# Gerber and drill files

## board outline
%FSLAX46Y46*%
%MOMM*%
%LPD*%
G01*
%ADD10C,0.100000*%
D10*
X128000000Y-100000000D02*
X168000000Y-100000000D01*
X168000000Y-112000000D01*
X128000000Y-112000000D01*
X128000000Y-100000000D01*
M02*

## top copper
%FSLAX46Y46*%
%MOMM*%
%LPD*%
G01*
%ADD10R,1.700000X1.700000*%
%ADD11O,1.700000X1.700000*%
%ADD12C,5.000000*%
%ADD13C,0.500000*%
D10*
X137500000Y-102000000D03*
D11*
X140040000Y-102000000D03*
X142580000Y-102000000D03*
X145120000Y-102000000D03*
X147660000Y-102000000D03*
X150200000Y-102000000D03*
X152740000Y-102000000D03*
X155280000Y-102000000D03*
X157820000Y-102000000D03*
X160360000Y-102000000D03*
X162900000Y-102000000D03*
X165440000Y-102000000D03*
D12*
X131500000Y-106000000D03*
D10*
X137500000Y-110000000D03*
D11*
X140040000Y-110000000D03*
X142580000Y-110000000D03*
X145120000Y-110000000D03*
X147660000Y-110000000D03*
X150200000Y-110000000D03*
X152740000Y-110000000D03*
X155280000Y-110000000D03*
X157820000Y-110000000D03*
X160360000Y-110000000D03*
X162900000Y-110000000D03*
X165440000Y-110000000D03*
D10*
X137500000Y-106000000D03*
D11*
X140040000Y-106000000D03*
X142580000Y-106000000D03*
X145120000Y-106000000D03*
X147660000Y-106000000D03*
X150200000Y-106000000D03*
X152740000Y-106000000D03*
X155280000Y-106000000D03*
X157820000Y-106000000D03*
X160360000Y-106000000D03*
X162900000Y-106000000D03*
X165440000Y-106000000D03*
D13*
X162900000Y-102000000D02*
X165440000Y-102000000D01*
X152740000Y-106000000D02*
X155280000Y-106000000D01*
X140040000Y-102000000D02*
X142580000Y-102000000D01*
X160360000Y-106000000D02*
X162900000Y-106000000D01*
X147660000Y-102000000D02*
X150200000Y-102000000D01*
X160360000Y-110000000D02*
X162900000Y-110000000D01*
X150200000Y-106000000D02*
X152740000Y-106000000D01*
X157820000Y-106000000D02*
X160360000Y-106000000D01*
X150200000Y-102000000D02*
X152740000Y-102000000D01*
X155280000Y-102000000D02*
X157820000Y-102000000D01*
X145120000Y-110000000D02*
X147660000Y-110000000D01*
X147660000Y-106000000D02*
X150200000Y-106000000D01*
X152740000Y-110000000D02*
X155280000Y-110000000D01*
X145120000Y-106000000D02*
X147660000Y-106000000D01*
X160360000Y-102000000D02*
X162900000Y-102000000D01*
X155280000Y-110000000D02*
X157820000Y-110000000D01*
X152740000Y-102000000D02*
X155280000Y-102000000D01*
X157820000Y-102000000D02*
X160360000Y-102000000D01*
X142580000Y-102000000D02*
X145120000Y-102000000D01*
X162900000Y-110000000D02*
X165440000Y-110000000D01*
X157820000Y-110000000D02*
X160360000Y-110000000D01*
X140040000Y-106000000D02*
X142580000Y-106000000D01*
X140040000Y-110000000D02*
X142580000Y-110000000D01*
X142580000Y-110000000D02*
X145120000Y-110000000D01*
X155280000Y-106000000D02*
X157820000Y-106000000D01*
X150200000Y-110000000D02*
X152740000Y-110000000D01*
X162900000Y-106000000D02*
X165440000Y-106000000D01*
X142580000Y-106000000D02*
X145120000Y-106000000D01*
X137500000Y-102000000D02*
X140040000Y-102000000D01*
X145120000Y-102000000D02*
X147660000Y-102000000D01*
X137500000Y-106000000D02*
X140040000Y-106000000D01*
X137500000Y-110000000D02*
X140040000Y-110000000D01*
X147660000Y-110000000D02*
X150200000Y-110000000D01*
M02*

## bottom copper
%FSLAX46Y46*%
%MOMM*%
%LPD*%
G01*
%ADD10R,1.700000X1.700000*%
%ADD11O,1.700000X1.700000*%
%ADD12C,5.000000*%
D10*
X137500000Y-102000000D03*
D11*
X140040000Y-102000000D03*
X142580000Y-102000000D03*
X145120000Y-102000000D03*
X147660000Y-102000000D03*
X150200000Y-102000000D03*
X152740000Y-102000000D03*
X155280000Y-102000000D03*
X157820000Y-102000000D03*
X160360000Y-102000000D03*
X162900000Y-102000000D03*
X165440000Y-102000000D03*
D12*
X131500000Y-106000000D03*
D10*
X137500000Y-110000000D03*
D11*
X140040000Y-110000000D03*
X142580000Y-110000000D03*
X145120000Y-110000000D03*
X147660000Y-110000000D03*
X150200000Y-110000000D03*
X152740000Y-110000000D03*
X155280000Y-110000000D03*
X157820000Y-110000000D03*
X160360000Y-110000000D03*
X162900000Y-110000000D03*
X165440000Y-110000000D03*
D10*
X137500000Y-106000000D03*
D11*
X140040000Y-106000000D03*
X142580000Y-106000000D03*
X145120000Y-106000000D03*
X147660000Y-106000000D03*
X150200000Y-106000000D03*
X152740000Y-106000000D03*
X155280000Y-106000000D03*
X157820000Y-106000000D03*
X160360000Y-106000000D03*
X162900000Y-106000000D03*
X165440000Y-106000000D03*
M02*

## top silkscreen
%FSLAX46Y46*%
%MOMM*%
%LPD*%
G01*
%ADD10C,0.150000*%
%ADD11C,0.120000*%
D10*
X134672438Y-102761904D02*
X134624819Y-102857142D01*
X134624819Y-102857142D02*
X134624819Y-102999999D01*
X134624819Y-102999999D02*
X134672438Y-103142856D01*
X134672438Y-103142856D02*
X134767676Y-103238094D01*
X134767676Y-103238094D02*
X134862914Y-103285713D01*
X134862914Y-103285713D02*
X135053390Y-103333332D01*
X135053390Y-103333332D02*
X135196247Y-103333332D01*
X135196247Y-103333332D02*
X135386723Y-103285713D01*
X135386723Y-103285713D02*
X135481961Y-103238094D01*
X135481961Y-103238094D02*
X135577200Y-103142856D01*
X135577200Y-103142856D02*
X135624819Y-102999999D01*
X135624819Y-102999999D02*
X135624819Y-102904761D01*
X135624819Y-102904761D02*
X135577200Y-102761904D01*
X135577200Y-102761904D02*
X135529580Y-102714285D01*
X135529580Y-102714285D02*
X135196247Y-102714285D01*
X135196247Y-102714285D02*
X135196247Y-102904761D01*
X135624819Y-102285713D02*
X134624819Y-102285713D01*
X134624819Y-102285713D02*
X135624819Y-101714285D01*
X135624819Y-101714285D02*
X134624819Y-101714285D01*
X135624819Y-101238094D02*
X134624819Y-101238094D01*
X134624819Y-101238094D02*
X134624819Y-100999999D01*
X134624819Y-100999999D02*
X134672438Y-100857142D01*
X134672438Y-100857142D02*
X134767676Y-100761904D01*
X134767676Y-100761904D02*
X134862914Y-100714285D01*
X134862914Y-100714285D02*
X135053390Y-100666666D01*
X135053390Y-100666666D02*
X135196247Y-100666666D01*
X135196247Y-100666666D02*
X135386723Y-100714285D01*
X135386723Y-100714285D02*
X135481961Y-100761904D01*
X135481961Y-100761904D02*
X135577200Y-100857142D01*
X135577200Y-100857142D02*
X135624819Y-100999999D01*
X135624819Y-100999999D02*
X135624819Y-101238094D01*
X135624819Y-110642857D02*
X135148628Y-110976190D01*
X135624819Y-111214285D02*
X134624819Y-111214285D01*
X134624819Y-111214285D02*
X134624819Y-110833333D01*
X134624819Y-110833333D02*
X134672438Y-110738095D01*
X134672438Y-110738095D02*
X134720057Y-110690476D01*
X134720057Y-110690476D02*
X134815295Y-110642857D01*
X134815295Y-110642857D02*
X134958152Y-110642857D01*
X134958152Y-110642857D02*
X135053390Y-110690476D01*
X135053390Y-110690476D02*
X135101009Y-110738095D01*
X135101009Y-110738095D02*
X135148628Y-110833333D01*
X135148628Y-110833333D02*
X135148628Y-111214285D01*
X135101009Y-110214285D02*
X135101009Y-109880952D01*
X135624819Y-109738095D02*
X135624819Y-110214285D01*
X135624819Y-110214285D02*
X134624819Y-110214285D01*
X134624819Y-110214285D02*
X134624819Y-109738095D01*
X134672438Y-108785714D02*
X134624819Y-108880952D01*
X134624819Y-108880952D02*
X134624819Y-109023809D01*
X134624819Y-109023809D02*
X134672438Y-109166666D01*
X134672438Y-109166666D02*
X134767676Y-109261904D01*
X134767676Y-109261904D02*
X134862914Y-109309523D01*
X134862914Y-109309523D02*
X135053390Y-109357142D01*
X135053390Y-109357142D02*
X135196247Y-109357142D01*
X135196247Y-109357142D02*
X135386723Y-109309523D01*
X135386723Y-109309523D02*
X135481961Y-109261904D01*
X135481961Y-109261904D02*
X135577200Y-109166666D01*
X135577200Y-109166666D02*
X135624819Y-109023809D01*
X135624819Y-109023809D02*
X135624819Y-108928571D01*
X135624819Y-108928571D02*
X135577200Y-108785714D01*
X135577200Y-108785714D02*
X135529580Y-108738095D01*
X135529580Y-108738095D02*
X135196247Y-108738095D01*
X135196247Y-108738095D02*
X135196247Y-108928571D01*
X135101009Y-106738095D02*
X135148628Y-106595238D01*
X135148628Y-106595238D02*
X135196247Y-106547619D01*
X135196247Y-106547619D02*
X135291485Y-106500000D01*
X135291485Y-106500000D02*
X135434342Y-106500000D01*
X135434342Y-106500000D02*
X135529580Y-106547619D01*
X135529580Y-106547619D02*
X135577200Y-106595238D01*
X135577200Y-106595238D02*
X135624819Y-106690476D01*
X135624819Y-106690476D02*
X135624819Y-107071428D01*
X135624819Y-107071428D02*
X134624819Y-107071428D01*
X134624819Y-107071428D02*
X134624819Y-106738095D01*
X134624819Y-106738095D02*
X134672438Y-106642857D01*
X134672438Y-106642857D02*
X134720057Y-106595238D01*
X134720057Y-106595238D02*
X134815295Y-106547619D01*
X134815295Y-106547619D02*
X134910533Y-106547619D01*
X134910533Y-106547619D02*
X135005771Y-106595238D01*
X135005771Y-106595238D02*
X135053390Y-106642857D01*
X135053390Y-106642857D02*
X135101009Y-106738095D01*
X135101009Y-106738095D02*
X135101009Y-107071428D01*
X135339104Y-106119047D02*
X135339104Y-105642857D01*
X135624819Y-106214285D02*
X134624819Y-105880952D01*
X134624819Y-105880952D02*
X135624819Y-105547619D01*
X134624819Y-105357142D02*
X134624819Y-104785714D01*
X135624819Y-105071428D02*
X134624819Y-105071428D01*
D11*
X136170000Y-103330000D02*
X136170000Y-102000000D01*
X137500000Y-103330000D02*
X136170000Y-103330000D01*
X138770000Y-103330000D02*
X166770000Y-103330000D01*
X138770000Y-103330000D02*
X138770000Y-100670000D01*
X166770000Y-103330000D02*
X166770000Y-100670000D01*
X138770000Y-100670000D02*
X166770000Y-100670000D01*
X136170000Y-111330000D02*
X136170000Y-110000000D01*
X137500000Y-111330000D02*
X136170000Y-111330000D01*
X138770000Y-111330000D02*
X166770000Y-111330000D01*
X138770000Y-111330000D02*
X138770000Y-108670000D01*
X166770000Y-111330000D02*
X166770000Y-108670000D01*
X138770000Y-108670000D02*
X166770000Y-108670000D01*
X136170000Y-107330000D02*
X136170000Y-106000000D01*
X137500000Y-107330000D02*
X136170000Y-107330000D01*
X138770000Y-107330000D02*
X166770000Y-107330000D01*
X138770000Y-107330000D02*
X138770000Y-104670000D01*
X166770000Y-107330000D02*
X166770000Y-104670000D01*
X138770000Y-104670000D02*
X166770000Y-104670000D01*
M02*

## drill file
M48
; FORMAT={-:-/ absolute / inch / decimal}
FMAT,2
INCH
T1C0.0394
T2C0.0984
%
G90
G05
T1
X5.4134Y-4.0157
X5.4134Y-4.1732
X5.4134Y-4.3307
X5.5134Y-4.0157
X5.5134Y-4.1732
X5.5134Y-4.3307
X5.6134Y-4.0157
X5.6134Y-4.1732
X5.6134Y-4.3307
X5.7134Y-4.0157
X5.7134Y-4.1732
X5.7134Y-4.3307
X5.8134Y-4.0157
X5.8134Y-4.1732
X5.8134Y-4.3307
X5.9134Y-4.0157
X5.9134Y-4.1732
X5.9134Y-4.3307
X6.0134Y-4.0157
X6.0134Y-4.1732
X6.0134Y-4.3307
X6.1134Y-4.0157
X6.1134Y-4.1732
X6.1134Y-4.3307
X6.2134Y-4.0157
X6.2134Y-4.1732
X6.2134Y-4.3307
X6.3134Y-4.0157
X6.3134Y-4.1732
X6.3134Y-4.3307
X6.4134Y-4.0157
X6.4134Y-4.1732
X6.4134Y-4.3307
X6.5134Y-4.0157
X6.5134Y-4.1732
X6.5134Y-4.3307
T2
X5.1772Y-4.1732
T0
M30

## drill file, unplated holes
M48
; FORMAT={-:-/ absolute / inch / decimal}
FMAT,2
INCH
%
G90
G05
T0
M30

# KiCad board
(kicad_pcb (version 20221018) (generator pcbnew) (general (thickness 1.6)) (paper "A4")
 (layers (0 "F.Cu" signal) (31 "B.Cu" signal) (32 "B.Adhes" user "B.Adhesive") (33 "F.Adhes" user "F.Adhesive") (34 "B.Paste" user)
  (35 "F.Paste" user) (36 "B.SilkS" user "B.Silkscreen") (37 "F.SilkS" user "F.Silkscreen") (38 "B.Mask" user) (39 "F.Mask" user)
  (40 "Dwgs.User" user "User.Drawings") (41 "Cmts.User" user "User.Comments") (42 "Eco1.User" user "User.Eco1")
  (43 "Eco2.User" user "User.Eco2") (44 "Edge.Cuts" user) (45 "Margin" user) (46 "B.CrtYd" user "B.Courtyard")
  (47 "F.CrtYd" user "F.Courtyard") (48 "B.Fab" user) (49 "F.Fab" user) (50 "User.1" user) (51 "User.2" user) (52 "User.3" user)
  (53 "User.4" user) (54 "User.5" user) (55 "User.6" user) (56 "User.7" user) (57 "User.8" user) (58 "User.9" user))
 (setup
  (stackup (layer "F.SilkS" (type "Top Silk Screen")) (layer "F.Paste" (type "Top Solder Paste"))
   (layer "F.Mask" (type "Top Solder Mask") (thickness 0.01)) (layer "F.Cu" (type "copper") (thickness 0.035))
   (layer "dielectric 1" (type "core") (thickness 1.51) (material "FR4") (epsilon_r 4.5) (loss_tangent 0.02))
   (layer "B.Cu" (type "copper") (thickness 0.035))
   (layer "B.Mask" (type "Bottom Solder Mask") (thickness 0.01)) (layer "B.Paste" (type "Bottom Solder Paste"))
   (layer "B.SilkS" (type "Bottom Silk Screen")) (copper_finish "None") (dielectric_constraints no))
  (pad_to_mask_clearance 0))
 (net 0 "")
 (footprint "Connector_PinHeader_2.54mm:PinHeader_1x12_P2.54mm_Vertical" (layer "F.Cu") (at 137.5 102 90)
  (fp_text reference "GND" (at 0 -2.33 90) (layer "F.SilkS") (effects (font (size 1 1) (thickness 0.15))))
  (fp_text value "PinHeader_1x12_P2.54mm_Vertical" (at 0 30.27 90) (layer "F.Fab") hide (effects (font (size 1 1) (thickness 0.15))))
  (fp_line (start -1.33 -1.33) (end 0 -1.33) (stroke (width 0.12) (type solid)) (layer "F.SilkS"))
  (fp_line (start -1.33 0) (end -1.33 -1.33) (stroke (width 0.12) (type solid)) (layer "F.SilkS"))
  (fp_line (start -1.33 1.27) (end -1.33 29.27) (stroke (width 0.12) (type solid)) (layer "F.SilkS"))
  (fp_line (start -1.33 1.27) (end 1.33 1.27) (stroke (width 0.12) (type solid)) (layer "F.SilkS"))
  (fp_line (start -1.33 29.27) (end 1.33 29.27) (stroke (width 0.12) (type solid)) (layer "F.SilkS"))
  (fp_line (start 1.33 1.27) (end 1.33 29.27) (stroke (width 0.12) (type solid)) (layer "F.SilkS"))
  (pad "1" thru_hole rect (at 0 0 90) (size 1.7 1.7) (drill 1) (layers "*.Cu" "*.Mask"))
  (pad "2" thru_hole oval (at 0 2.54 90) (size 1.7 1.7) (drill 1) (layers "*.Cu" "*.Mask"))
  (pad "3" thru_hole oval (at 0 5.08 90) (size 1.7 1.7) (drill 1) (layers "*.Cu" "*.Mask"))
  (pad "4" thru_hole oval (at 0 7.62 90) (size 1.7 1.7) (drill 1) (layers "*.Cu" "*.Mask"))
  (pad "5" thru_hole oval (at 0 10.16 90) (size 1.7 1.7) (drill 1) (layers "*.Cu" "*.Mask"))
  (pad "6" thru_hole oval (at 0 12.7 90) (size 1.7 1.7) (drill 1) (layers "*.Cu" "*.Mask"))
  (pad "7" thru_hole oval (at 0 15.24 90) (size 1.7 1.7) (drill 1) (layers "*.Cu" "*.Mask"))
  (pad "8" thru_hole oval (at 0 17.78 90) (size 1.7 1.7) (drill 1) (layers "*.Cu" "*.Mask"))
  (pad "9" thru_hole oval (at 0 20.32 90) (size 1.7 1.7) (drill 1) (layers "*.Cu" "*.Mask"))
  (pad "10" thru_hole oval (at 0 22.86 90) (size 1.7 1.7) (drill 1) (layers "*.Cu" "*.Mask"))
  (pad "11" thru_hole oval (at 0 25.4 90) (size 1.7 1.7) (drill 1) (layers "*.Cu" "*.Mask"))
  (pad "12" thru_hole oval (at 0 27.94 90) (size 1.7 1.7) (drill 1) (layers "*.Cu" "*.Mask")))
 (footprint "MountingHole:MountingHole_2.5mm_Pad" (layer "F.Cu") (at 131.5 106)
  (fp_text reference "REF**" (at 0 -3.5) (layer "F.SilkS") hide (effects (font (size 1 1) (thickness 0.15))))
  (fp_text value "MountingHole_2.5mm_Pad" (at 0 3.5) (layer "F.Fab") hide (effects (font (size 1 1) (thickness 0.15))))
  (pad "1" thru_hole circle (at 0 0) (size 5 5) (drill 2.5) (layers "*.Cu" "*.Mask")))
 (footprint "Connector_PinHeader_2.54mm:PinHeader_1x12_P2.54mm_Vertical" (layer "F.Cu") (at 137.5 110 90)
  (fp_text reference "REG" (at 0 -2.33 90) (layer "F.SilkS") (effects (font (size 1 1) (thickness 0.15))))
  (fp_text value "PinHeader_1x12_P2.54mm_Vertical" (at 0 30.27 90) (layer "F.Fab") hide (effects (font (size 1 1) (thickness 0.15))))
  (fp_line (start -1.33 -1.33) (end 0 -1.33) (stroke (width 0.12) (type solid)) (layer "F.SilkS"))
  (fp_line (start -1.33 0) (end -1.33 -1.33) (stroke (width 0.12) (type solid)) (layer "F.SilkS"))
  (fp_line (start -1.33 1.27) (end -1.33 29.27) (stroke (width 0.12) (type solid)) (layer "F.SilkS"))
  (fp_line (start -1.33 1.27) (end 1.33 1.27) (stroke (width 0.12) (type solid)) (layer "F.SilkS"))
  (fp_line (start -1.33 29.27) (end 1.33 29.27) (stroke (width 0.12) (type solid)) (layer "F.SilkS"))
  (fp_line (start 1.33 1.27) (end 1.33 29.27) (stroke (width 0.12) (type solid)) (layer "F.SilkS"))
  (pad "1" thru_hole rect (at 0 0 90) (size 1.7 1.7) (drill 1) (layers "*.Cu" "*.Mask"))
  (pad "2" thru_hole oval (at 0 2.54 90) (size 1.7 1.7) (drill 1) (layers "*.Cu" "*.Mask"))
  (pad "3" thru_hole oval (at 0 5.08 90) (size 1.7 1.7) (drill 1) (layers "*.Cu" "*.Mask"))
  (pad "4" thru_hole oval (at 0 7.62 90) (size 1.7 1.7) (drill 1) (layers "*.Cu" "*.Mask"))
  (pad "5" thru_hole oval (at 0 10.16 90) (size 1.7 1.7) (drill 1) (layers "*.Cu" "*.Mask"))
  (pad "6" thru_hole oval (at 0 12.7 90) (size 1.7 1.7) (drill 1) (layers "*.Cu" "*.Mask"))
  (pad "7" thru_hole oval (at 0 15.24 90) (size 1.7 1.7) (drill 1) (layers "*.Cu" "*.Mask"))
  (pad "8" thru_hole oval (at 0 17.78 90) (size 1.7 1.7) (drill 1) (layers "*.Cu" "*.Mask"))
  (pad "9" thru_hole oval (at 0 20.32 90) (size 1.7 1.7) (drill 1) (layers "*.Cu" "*.Mask"))
  (pad "10" thru_hole oval (at 0 22.86 90) (size 1.7 1.7) (drill 1) (layers "*.Cu" "*.Mask"))
  (pad "11" thru_hole oval (at 0 25.4 90) (size 1.7 1.7) (drill 1) (layers "*.Cu" "*.Mask"))
  (pad "12" thru_hole oval (at 0 27.94 90) (size 1.7 1.7) (drill 1) (layers "*.Cu" "*.Mask")))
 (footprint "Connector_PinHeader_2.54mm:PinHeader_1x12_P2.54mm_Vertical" (layer "F.Cu") (at 137.5 106 90)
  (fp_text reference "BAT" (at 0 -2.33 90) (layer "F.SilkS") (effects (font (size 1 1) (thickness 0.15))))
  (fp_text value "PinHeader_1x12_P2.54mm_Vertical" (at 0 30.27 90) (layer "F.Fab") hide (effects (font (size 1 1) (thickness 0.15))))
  (fp_line (start -1.33 -1.33) (end 0 -1.33) (stroke (width 0.12) (type solid)) (layer "F.SilkS"))
  (fp_line (start -1.33 0) (end -1.33 -1.33) (stroke (width 0.12) (type solid)) (layer "F.SilkS"))
  (fp_line (start -1.33 1.27) (end -1.33 29.27) (stroke (width 0.12) (type solid)) (layer "F.SilkS"))
  (fp_line (start -1.33 1.27) (end 1.33 1.27) (stroke (width 0.12) (type solid)) (layer "F.SilkS"))
  (fp_line (start -1.33 29.27) (end 1.33 29.27) (stroke (width 0.12) (type solid)) (layer "F.SilkS"))
  (fp_line (start 1.33 1.27) (end 1.33 29.27) (stroke (width 0.12) (type solid)) (layer "F.SilkS"))
  (pad "1" thru_hole rect (at 0 0 90) (size 1.7 1.7) (drill 1) (layers "*.Cu" "*.Mask"))
  (pad "2" thru_hole oval (at 0 2.54 90) (size 1.7 1.7) (drill 1) (layers "*.Cu" "*.Mask"))
  (pad "3" thru_hole oval (at 0 5.08 90) (size 1.7 1.7) (drill 1) (layers "*.Cu" "*.Mask"))
  (pad "4" thru_hole oval (at 0 7.62 90) (size 1.7 1.7) (drill 1) (layers "*.Cu" "*.Mask"))
  (pad "5" thru_hole oval (at 0 10.16 90) (size 1.7 1.7) (drill 1) (layers "*.Cu" "*.Mask"))
  (pad "6" thru_hole oval (at 0 12.7 90) (size 1.7 1.7) (drill 1) (layers "*.Cu" "*.Mask"))
  (pad "7" thru_hole oval (at 0 15.24 90) (size 1.7 1.7) (drill 1) (layers "*.Cu" "*.Mask"))
  (pad "8" thru_hole oval (at 0 17.78 90) (size 1.7 1.7) (drill 1) (layers "*.Cu" "*.Mask"))
  (pad "9" thru_hole oval (at 0 20.32 90) (size 1.7 1.7) (drill 1) (layers "*.Cu" "*.Mask"))
  (pad "10" thru_hole oval (at 0 22.86 90) (size 1.7 1.7) (drill 1) (layers "*.Cu" "*.Mask"))
  (pad "11" thru_hole oval (at 0 25.4 90) (size 1.7 1.7) (drill 1) (layers "*.Cu" "*.Mask"))
  (pad "12" thru_hole oval (at 0 27.94 90) (size 1.7 1.7) (drill 1) (layers "*.Cu" "*.Mask")))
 (gr_rect (start 128 100) (end 168 112) (stroke (width 0.1) (type default)) (fill none) (layer "Edge.Cuts"))
 (segment (start 162.9 102) (end 165.44 102) (width 0.5) (layer "F.Cu") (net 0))
 (segment (start 152.74 106) (end 155.28 106) (width 0.5) (layer "F.Cu") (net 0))
 (segment (start 140.04 102) (end 142.58 102) (width 0.5) (layer "F.Cu") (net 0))
 (segment (start 160.36 106) (end 162.9 106) (width 0.5) (layer "F.Cu") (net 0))
 (segment (start 147.66 102) (end 150.2 102) (width 0.5) (layer "F.Cu") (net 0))
 (segment (start 160.36 110) (end 162.9 110) (width 0.5) (layer "F.Cu") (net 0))
 (segment (start 150.2 106) (end 152.74 106) (width 0.5) (layer "F.Cu") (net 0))
 (segment (start 157.82 106) (end 160.36 106) (width 0.5) (layer "F.Cu") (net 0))
 (segment (start 150.2 102) (end 152.74 102) (width 0.5) (layer "F.Cu") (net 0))
 (segment (start 155.28 102) (end 157.82 102) (width 0.5) (layer "F.Cu") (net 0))
 (segment (start 145.12 110) (end 147.66 110) (width 0.5) (layer "F.Cu") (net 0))
 (segment (start 147.66 106) (end 150.2 106) (width 0.5) (layer "F.Cu") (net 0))
 (segment (start 152.74 110) (end 155.28 110) (width 0.5) (layer "F.Cu") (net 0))
 (segment (start 145.12 106) (end 147.66 106) (width 0.5) (layer "F.Cu") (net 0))
 (segment (start 160.36 102) (end 162.9 102) (width 0.5) (layer "F.Cu") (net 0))
 (segment (start 155.28 110) (end 157.82 110) (width 0.5) (layer "F.Cu") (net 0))
 (segment (start 152.74 102) (end 155.28 102) (width 0.5) (layer "F.Cu") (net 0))
 (segment (start 157.82 102) (end 160.36 102) (width 0.5) (layer "F.Cu") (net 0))
 (segment (start 142.58 102) (end 145.12 102) (width 0.5) (layer "F.Cu") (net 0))
 (segment (start 162.9 110) (end 165.44 110) (width 0.5) (layer "F.Cu") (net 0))
 (segment (start 157.82 110) (end 160.36 110) (width 0.5) (layer "F.Cu") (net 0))
 (segment (start 140.04 106) (end 142.58 106) (width 0.5) (layer "F.Cu") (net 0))
 (segment (start 140.04 110) (end 142.58 110) (width 0.5) (layer "F.Cu") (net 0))
 (segment (start 142.58 110) (end 145.12 110) (width 0.5) (layer "F.Cu") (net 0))
 (segment (start 155.28 106) (end 157.82 106) (width 0.5) (layer "F.Cu") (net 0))
 (segment (start 150.2 110) (end 152.74 110) (width 0.5) (layer "F.Cu") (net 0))
 (segment (start 162.9 106) (end 165.44 106) (width 0.5) (layer "F.Cu") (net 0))
 (segment (start 142.58 106) (end 145.12 106) (width 0.5) (layer "F.Cu") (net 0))
 (segment (start 137.5 102) (end 140.04 102) (width 0.5) (layer "F.Cu") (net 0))
 (segment (start 145.12 102) (end 147.66 102) (width 0.5) (layer "F.Cu") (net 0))
 (segment (start 137.5 106) (end 140.04 106) (width 0.5) (layer "F.Cu") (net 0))
 (segment (start 137.5 110) (end 140.04 110) (width 0.5) (layer "F.Cu") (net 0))
 (segment (start 147.66 110) (end 150.2 110) (width 0.5) (layer "F.Cu") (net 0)))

